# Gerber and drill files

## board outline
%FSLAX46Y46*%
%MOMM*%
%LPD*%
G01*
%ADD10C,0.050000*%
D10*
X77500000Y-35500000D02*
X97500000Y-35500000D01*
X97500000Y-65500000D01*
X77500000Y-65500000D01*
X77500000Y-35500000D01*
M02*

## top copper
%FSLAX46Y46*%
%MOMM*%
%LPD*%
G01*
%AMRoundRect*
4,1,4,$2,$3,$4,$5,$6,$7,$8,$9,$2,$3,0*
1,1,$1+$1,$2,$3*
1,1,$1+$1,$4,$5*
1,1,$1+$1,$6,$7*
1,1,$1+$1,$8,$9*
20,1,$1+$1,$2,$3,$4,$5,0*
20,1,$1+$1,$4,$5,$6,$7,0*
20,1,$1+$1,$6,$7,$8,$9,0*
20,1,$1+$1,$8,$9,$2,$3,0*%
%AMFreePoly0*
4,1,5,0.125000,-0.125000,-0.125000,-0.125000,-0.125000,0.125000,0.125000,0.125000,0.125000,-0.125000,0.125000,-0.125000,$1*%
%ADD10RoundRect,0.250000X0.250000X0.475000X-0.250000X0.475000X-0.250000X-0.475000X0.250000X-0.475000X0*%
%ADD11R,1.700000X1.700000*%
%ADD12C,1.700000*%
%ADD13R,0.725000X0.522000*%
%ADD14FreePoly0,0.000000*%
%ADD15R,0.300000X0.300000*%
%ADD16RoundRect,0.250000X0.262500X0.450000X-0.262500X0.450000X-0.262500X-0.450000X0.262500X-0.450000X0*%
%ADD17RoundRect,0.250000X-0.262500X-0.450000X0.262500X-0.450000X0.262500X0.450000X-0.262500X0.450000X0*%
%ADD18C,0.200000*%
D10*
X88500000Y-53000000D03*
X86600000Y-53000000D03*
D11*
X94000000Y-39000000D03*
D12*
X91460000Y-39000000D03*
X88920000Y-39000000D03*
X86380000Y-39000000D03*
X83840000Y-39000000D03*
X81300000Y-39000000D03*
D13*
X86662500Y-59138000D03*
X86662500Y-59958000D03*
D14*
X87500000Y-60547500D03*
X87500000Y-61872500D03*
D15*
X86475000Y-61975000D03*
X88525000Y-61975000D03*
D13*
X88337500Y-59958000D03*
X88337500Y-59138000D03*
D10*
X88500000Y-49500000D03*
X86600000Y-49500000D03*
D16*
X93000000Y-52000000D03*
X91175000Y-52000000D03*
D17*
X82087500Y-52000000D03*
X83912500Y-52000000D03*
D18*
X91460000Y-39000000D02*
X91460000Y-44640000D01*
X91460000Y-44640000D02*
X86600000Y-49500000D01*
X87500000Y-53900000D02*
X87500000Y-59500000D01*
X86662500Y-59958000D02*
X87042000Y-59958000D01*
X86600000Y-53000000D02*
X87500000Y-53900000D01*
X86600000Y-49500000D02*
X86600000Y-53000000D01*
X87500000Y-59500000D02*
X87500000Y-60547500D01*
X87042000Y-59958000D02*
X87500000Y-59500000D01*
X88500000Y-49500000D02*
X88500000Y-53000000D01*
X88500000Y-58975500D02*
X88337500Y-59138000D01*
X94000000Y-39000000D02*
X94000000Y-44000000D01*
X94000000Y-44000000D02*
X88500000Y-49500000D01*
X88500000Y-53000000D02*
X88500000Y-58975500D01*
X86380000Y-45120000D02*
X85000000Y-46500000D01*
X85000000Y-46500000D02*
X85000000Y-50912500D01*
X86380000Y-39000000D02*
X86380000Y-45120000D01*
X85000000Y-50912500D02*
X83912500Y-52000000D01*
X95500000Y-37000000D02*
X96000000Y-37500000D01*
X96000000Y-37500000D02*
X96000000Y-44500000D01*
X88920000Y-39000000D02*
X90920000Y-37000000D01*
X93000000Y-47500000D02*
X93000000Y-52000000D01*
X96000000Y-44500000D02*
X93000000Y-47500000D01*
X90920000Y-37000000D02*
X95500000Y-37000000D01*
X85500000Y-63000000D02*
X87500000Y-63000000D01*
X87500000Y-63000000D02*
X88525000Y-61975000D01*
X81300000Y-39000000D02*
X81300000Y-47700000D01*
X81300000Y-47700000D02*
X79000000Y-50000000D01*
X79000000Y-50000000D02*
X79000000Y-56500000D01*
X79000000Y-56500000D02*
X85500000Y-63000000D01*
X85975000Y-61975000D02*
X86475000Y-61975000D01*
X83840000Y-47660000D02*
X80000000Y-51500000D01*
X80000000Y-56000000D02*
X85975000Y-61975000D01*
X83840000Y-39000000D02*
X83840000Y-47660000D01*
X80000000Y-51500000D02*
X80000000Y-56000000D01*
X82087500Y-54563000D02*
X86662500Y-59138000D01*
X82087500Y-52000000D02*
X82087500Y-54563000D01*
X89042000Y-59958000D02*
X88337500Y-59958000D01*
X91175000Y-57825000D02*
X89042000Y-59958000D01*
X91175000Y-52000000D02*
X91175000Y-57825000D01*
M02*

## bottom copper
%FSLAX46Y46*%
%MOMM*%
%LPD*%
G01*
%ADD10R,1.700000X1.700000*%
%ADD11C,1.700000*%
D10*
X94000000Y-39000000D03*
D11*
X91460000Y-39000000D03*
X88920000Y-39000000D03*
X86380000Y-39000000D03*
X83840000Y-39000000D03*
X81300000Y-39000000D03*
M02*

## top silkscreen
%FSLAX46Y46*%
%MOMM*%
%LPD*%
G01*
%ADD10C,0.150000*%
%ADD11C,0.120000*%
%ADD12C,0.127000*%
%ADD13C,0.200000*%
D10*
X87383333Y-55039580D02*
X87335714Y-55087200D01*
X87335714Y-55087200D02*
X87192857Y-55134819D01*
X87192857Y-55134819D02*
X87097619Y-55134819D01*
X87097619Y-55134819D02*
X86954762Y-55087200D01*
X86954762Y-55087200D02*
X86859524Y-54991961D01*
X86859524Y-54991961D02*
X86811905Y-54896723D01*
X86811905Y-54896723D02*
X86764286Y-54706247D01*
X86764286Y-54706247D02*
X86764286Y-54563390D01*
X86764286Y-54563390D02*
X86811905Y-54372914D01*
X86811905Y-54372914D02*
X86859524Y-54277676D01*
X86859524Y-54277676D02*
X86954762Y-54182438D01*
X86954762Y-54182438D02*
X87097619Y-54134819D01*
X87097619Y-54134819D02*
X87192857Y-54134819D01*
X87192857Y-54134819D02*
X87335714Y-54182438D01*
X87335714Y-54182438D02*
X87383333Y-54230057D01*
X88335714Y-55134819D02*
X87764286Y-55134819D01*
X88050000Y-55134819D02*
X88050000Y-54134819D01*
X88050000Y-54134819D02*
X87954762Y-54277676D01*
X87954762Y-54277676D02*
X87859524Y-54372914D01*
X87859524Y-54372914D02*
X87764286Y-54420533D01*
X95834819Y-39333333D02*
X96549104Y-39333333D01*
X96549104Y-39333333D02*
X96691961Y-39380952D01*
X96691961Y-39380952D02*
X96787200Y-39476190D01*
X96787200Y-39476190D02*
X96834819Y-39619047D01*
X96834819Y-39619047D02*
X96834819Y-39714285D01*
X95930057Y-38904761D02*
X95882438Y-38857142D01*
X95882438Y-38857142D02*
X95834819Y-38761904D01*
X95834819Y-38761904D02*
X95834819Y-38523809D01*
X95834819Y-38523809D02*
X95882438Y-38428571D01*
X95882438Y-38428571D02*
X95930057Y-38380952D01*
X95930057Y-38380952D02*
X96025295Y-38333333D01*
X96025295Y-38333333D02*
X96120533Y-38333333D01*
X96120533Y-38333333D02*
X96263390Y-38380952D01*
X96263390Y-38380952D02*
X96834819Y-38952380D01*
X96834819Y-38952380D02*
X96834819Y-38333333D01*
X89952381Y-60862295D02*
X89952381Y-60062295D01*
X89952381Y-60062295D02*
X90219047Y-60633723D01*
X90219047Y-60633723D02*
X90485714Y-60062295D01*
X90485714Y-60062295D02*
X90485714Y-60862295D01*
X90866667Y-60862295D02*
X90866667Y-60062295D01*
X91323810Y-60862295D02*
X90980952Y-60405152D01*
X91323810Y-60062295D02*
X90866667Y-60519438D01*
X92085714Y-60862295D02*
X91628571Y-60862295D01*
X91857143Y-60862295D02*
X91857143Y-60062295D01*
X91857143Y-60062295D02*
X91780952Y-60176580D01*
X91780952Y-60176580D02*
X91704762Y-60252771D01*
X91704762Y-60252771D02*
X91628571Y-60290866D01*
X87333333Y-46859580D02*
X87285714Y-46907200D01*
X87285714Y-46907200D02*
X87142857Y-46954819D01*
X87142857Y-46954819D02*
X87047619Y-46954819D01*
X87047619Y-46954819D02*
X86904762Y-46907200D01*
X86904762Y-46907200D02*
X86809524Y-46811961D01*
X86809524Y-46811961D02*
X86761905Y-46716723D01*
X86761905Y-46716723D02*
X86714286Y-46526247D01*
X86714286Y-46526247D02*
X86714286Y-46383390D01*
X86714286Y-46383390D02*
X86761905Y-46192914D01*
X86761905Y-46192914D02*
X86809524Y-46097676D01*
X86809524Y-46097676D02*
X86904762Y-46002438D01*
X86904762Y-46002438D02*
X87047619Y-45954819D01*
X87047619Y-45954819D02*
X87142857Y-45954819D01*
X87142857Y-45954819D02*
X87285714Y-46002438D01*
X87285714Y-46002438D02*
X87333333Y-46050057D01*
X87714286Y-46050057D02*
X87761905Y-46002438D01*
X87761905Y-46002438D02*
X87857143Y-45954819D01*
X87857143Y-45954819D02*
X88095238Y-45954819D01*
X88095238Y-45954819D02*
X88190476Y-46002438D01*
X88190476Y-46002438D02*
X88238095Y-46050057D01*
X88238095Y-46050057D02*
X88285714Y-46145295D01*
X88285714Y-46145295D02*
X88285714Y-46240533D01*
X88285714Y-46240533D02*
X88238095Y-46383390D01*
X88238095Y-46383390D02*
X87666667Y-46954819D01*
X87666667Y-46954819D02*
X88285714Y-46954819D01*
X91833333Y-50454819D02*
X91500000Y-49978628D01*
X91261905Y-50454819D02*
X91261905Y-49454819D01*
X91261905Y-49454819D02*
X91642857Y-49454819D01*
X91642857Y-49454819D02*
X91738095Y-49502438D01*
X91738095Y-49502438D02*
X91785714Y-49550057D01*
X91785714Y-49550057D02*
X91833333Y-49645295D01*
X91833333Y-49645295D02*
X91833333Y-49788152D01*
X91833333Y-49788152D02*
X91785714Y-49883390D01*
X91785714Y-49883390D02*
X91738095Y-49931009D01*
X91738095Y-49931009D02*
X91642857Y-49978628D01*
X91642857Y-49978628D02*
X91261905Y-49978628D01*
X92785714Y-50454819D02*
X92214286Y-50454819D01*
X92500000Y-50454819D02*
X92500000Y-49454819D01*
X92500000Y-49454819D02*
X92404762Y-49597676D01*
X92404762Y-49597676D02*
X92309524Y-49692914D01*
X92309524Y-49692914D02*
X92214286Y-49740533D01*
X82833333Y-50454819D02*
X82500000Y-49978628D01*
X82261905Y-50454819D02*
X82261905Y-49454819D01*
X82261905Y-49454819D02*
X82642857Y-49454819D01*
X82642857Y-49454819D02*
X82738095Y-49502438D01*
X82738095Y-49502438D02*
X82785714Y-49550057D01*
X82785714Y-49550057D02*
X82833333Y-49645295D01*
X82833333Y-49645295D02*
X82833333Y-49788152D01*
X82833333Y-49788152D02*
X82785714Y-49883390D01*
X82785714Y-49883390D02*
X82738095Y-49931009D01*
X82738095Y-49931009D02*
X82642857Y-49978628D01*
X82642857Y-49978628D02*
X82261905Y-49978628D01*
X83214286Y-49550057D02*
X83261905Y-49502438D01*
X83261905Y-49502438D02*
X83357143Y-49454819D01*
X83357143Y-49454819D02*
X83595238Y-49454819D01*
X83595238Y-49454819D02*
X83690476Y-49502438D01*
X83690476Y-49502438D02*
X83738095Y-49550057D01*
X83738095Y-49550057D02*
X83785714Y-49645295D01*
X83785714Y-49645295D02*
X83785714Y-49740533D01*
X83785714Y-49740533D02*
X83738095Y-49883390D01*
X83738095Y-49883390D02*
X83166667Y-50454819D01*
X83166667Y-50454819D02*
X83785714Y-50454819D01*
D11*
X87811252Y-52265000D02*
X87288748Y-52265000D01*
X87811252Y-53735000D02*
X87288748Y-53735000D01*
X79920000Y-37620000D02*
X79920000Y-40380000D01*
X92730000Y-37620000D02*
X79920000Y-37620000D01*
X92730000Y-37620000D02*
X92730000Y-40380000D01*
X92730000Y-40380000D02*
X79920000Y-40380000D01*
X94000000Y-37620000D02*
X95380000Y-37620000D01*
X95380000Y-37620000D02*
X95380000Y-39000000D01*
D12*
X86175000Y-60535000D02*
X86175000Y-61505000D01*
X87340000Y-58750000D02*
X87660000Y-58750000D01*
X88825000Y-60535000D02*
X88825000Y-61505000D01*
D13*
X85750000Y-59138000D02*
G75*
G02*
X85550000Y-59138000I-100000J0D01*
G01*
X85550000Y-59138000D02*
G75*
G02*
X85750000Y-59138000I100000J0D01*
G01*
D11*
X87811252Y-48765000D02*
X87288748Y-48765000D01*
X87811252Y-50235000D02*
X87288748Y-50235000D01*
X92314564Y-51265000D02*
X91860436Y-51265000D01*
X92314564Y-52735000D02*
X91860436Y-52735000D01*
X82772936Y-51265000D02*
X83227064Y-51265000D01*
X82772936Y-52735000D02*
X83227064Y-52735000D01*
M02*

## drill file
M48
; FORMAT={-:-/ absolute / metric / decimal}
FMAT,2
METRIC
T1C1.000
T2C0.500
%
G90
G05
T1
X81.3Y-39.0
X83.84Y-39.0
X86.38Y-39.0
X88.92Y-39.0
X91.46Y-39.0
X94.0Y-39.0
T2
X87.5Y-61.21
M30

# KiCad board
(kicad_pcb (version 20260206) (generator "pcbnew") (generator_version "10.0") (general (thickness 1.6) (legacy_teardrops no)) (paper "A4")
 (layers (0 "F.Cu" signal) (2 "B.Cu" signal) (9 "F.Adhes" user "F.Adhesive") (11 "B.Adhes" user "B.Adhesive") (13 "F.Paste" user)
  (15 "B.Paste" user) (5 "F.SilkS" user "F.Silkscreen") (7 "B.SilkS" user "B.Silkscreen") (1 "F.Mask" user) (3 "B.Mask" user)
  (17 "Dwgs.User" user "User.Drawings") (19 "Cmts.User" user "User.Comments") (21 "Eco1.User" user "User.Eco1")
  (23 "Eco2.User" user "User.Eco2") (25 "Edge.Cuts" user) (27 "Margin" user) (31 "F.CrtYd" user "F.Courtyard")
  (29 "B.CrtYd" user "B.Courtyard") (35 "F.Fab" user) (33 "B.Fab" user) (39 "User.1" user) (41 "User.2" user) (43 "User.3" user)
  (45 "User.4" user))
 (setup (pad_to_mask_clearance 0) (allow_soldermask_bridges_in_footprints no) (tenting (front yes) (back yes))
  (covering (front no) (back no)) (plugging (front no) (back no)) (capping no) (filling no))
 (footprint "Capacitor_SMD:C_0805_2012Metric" (layer "F.Cu") (at 87.55 53 180)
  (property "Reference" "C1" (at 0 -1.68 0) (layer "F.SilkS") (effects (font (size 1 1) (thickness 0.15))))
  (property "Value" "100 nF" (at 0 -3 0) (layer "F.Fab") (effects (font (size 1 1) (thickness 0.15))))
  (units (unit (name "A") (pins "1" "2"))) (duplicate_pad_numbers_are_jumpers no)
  (fp_line (start -0.261252 0.735) (end 0.261252 0.735) (stroke (width 0.12) (type solid)) (layer "F.SilkS"))
  (fp_line (start -0.261252 -0.735) (end 0.261252 -0.735) (stroke (width 0.12) (type solid)) (layer "F.SilkS"))
  (pad "1" smd roundrect (at -0.95 0 180) (size 1 1.45) (layers "F.Cu" "F.Mask" "F.Paste") (roundrect_rratio 0.25) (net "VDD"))
  (pad "2" smd roundrect (at 0.95 0 180) (size 1 1.45) (layers "F.Cu" "F.Mask" "F.Paste") (roundrect_rratio 0.25) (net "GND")))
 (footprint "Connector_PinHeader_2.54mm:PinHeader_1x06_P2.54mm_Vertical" (layer "F.Cu") (at 94 39 -90)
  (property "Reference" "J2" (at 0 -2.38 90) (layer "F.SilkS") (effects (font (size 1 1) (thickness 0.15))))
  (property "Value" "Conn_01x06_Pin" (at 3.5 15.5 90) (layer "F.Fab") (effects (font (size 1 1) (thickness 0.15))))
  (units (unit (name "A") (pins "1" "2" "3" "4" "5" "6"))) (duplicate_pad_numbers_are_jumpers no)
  (fp_line (start -1.38 14.08) (end 1.38 14.08) (stroke (width 0.12) (type solid)) (layer "F.SilkS"))
  (fp_line (start -1.38 1.27) (end -1.38 14.08) (stroke (width 0.12) (type solid)) (layer "F.SilkS"))
  (fp_line (start -1.38 1.27) (end 1.38 1.27) (stroke (width 0.12) (type solid)) (layer "F.SilkS"))
  (fp_line (start 1.38 1.27) (end 1.38 14.08) (stroke (width 0.12) (type solid)) (layer "F.SilkS"))
  (fp_line (start -1.38 0) (end -1.38 -1.38) (stroke (width 0.12) (type solid)) (layer "F.SilkS"))
  (fp_line (start -1.38 -1.38) (end 0 -1.38) (stroke (width 0.12) (type solid)) (layer "F.SilkS"))
  (pad "1" thru_hole rect (at 0 0 270) (size 1.7 1.7) (drill 1) (layers "*.Cu" "*.Mask") (remove_unused_layers no) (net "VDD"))
  (pad "2" thru_hole circle (at 0 2.54 270) (size 1.7 1.7) (drill 1) (layers "*.Cu" "*.Mask") (remove_unused_layers no) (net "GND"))
  (pad "3" thru_hole circle (at 0 5.08 270) (size 1.7 1.7) (drill 1) (layers "*.Cu" "*.Mask") (remove_unused_layers no)
   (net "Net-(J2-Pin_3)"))
  (pad "4" thru_hole circle (at 0 7.62 270) (size 1.7 1.7) (drill 1) (layers "*.Cu" "*.Mask") (remove_unused_layers no)
   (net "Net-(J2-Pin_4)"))
  (pad "5" thru_hole circle (at 0 10.16 270) (size 1.7 1.7) (drill 1) (layers "*.Cu" "*.Mask") (remove_unused_layers no)
   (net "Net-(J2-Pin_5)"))
  (pad "6" thru_hole circle (at 0 12.7 270) (size 1.7 1.7) (drill 1) (layers "*.Cu" "*.Mask") (remove_unused_layers no)
   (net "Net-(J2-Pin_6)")))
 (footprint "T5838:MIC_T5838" (layer "F.Cu") (at 87.5 60.5)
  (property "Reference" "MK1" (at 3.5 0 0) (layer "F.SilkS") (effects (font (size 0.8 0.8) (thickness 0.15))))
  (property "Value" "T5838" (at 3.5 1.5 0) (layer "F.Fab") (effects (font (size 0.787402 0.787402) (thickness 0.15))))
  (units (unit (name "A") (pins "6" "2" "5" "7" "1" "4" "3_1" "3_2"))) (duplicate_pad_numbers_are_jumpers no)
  (fp_line (start -1.325 0.035) (end -1.325 1.005) (stroke (width 0.127) (type solid)) (layer "F.SilkS"))
  (fp_line (start -0.16 -1.75) (end 0.16 -1.75) (stroke (width 0.127) (type solid)) (layer "F.SilkS"))
  (fp_line (start 1.325 0.035) (end 1.325 1.005) (stroke (width 0.127) (type solid)) (layer "F.SilkS"))
  (fp_circle (center -1.85 -1.362) (end -1.75 -1.362) (stroke (width 0.2) (type solid)) (fill no) (layer "F.SilkS"))
  (pad "" np_thru_hole circle (at 0 0.71) (size 0.5 0.5) (drill 0.5) (layers "*.Cu" "*.Mask"))
  (pad "1" smd rect (at -0.8375 -1.362) (size 0.725 0.522) (layers "F.Cu") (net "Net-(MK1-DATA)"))
  (pad "2" smd rect (at -0.8375 -0.542) (size 0.725 0.522) (layers "F.Cu") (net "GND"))
  (pad "3_1" smd custom (at 0 0.0475) (size 0.25 0.25) (layers "F.Cu") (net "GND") (options (clearance outline) (anchor rect)) (primitives))
  (pad "3_2" smd custom (at 0 1.3725) (size 0.25 0.25) (layers "F.Cu") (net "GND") (options (clearance outline) (anchor rect)) (primitives))
  (pad "4" smd rect (at -1.025 1.475) (size 0.3 0.3) (layers "F.Cu") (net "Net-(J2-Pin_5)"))
  (pad "5" smd rect (at 1.025 1.475) (size 0.3 0.3) (layers "F.Cu") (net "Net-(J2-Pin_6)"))
  (pad "6" smd rect (at 0.8375 -0.542) (size 0.725 0.522) (layers "F.Cu") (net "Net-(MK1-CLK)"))
  (pad "7" smd rect (at 0.8375 -1.362) (size 0.725 0.522) (layers "F.Cu") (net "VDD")))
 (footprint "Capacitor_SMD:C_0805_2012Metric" (layer "F.Cu") (at 87.55 49.5 180)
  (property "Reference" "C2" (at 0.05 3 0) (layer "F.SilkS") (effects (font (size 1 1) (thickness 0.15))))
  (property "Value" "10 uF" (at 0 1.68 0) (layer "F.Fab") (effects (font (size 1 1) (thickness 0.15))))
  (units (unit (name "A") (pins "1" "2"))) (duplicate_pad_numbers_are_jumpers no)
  (fp_line (start -0.261252 0.735) (end 0.261252 0.735) (stroke (width 0.12) (type solid)) (layer "F.SilkS"))
  (fp_line (start -0.261252 -0.735) (end 0.261252 -0.735) (stroke (width 0.12) (type solid)) (layer "F.SilkS"))
  (pad "1" smd roundrect (at -0.95 0 180) (size 1 1.45) (layers "F.Cu" "F.Mask" "F.Paste") (roundrect_rratio 0.25) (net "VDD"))
  (pad "2" smd roundrect (at 0.95 0 180) (size 1 1.45) (layers "F.Cu" "F.Mask" "F.Paste") (roundrect_rratio 0.25) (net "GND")))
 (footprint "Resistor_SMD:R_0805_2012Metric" (layer "F.Cu") (at 92.0875 52 180)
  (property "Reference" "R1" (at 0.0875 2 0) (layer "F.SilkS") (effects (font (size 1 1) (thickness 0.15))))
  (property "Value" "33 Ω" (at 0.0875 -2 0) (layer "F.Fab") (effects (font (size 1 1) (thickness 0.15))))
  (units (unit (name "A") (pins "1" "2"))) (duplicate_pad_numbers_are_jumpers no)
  (fp_line (start -0.227064 0.735) (end 0.227064 0.735) (stroke (width 0.12) (type solid)) (layer "F.SilkS"))
  (fp_line (start -0.227064 -0.735) (end 0.227064 -0.735) (stroke (width 0.12) (type solid)) (layer "F.SilkS"))
  (pad "1" smd roundrect (at -0.9125 0 180) (size 1.025 1.4) (layers "F.Cu" "F.Mask" "F.Paste") (roundrect_rratio 0.243902)
   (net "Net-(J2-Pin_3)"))
  (pad "2" smd roundrect (at 0.9125 0 180) (size 1.025 1.4) (layers "F.Cu" "F.Mask" "F.Paste") (roundrect_rratio 0.243902)
   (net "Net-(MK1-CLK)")))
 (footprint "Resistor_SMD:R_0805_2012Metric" (layer "F.Cu") (at 83 52)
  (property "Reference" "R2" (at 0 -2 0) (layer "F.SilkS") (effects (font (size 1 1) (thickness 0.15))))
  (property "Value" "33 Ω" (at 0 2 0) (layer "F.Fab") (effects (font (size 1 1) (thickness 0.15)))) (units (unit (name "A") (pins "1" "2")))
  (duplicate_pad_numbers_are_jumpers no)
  (fp_line (start -0.227064 -0.735) (end 0.227064 -0.735) (stroke (width 0.12) (type solid)) (layer "F.SilkS"))
  (fp_line (start -0.227064 0.735) (end 0.227064 0.735) (stroke (width 0.12) (type solid)) (layer "F.SilkS"))
  (pad "1" smd roundrect (at -0.9125 0) (size 1.025 1.4) (layers "F.Cu" "F.Mask" "F.Paste") (roundrect_rratio 0.243902)
   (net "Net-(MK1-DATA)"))
  (pad "2" smd roundrect (at 0.9125 0) (size 1.025 1.4) (layers "F.Cu" "F.Mask" "F.Paste") (roundrect_rratio 0.243902)
   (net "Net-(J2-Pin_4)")))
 (gr_rect (start 77.5 35.5) (end 97.5 65.5) (stroke (width 0.05) (type default)) (fill no) (layer "Edge.Cuts"))
 (segment (start 91.46 39) (end 91.46 44.64) (width 0.2) (layer "F.Cu") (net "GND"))
 (segment (start 91.46 44.64) (end 86.6 49.5) (width 0.2) (layer "F.Cu") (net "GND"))
 (segment (start 87.5 53.9) (end 87.5 59.5) (width 0.2) (layer "F.Cu") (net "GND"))
 (segment (start 86.6625 59.958) (end 87.042 59.958) (width 0.2) (layer "F.Cu") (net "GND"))
 (segment (start 86.6 53) (end 87.5 53.9) (width 0.2) (layer "F.Cu") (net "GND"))
 (segment (start 86.6 49.5) (end 86.6 53) (width 0.2) (layer "F.Cu") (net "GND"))
 (segment (start 87.5 59.5) (end 87.5 60.5475) (width 0.2) (layer "F.Cu") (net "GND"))
 (segment (start 87.042 59.958) (end 87.5 59.5) (width 0.2) (layer "F.Cu") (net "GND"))
 (segment (start 88.5 49.5) (end 88.5 53) (width 0.2) (layer "F.Cu") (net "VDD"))
 (segment (start 88.5 58.9755) (end 88.3375 59.138) (width 0.2) (layer "F.Cu") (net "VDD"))
 (segment (start 94 39) (end 94 44) (width 0.2) (layer "F.Cu") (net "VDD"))
 (segment (start 94 44) (end 88.5 49.5) (width 0.2) (layer "F.Cu") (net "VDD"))
 (segment (start 88.5 53) (end 88.5 58.9755) (width 0.2) (layer "F.Cu") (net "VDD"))
 (segment (start 86.38 45.12) (end 85 46.5) (width 0.2) (layer "F.Cu") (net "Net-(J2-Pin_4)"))
 (segment (start 85 46.5) (end 85 50.9125) (width 0.2) (layer "F.Cu") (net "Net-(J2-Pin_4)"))
 (segment (start 86.38 39) (end 86.38 45.12) (width 0.2) (layer "F.Cu") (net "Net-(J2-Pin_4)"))
 (segment (start 85 50.9125) (end 83.9125 52) (width 0.2) (layer "F.Cu") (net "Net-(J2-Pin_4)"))
 (segment (start 95.5 37) (end 96 37.5) (width 0.2) (layer "F.Cu") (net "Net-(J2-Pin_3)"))
 (segment (start 96 37.5) (end 96 44.5) (width 0.2) (layer "F.Cu") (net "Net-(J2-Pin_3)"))
 (segment (start 88.92 39) (end 90.92 37) (width 0.2) (layer "F.Cu") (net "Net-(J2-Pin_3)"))
 (segment (start 93 47.5) (end 93 52) (width 0.2) (layer "F.Cu") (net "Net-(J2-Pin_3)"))
 (segment (start 96 44.5) (end 93 47.5) (width 0.2) (layer "F.Cu") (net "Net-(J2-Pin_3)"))
 (segment (start 90.92 37) (end 95.5 37) (width 0.2) (layer "F.Cu") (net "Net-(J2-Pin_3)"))
 (segment (start 85.5 63) (end 87.5 63) (width 0.2) (layer "F.Cu") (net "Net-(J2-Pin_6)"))
 (segment (start 87.5 63) (end 88.525 61.975) (width 0.2) (layer "F.Cu") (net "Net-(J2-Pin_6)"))
 (segment (start 81.3 39) (end 81.3 47.7) (width 0.2) (layer "F.Cu") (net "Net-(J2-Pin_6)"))
 (segment (start 81.3 47.7) (end 79 50) (width 0.2) (layer "F.Cu") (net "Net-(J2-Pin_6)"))
 (segment (start 79 50) (end 79 56.5) (width 0.2) (layer "F.Cu") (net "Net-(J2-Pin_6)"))
 (segment (start 79 56.5) (end 85.5 63) (width 0.2) (layer "F.Cu") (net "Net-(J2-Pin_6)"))
 (segment (start 85.975 61.975) (end 86.475 61.975) (width 0.2) (layer "F.Cu") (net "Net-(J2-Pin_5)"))
 (segment (start 83.84 47.66) (end 80 51.5) (width 0.2) (layer "F.Cu") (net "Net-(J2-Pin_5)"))
 (segment (start 80 56) (end 85.975 61.975) (width 0.2) (layer "F.Cu") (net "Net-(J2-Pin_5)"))
 (segment (start 83.84 39) (end 83.84 47.66) (width 0.2) (layer "F.Cu") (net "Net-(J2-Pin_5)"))
 (segment (start 80 51.5) (end 80 56) (width 0.2) (layer "F.Cu") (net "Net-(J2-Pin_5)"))
 (segment (start 82.0875 54.563) (end 86.6625 59.138) (width 0.2) (layer "F.Cu") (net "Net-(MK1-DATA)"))
 (segment (start 82.0875 52) (end 82.0875 54.563) (width 0.2) (layer "F.Cu") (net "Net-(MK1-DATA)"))
 (segment (start 89.042 59.958) (end 88.3375 59.958) (width 0.2) (layer "F.Cu") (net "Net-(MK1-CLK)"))
 (segment (start 91.175 57.825) (end 89.042 59.958) (width 0.2) (layer "F.Cu") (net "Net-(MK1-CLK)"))
 (segment (start 91.175 52) (end 91.175 57.825) (width 0.2) (layer "F.Cu") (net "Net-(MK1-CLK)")))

